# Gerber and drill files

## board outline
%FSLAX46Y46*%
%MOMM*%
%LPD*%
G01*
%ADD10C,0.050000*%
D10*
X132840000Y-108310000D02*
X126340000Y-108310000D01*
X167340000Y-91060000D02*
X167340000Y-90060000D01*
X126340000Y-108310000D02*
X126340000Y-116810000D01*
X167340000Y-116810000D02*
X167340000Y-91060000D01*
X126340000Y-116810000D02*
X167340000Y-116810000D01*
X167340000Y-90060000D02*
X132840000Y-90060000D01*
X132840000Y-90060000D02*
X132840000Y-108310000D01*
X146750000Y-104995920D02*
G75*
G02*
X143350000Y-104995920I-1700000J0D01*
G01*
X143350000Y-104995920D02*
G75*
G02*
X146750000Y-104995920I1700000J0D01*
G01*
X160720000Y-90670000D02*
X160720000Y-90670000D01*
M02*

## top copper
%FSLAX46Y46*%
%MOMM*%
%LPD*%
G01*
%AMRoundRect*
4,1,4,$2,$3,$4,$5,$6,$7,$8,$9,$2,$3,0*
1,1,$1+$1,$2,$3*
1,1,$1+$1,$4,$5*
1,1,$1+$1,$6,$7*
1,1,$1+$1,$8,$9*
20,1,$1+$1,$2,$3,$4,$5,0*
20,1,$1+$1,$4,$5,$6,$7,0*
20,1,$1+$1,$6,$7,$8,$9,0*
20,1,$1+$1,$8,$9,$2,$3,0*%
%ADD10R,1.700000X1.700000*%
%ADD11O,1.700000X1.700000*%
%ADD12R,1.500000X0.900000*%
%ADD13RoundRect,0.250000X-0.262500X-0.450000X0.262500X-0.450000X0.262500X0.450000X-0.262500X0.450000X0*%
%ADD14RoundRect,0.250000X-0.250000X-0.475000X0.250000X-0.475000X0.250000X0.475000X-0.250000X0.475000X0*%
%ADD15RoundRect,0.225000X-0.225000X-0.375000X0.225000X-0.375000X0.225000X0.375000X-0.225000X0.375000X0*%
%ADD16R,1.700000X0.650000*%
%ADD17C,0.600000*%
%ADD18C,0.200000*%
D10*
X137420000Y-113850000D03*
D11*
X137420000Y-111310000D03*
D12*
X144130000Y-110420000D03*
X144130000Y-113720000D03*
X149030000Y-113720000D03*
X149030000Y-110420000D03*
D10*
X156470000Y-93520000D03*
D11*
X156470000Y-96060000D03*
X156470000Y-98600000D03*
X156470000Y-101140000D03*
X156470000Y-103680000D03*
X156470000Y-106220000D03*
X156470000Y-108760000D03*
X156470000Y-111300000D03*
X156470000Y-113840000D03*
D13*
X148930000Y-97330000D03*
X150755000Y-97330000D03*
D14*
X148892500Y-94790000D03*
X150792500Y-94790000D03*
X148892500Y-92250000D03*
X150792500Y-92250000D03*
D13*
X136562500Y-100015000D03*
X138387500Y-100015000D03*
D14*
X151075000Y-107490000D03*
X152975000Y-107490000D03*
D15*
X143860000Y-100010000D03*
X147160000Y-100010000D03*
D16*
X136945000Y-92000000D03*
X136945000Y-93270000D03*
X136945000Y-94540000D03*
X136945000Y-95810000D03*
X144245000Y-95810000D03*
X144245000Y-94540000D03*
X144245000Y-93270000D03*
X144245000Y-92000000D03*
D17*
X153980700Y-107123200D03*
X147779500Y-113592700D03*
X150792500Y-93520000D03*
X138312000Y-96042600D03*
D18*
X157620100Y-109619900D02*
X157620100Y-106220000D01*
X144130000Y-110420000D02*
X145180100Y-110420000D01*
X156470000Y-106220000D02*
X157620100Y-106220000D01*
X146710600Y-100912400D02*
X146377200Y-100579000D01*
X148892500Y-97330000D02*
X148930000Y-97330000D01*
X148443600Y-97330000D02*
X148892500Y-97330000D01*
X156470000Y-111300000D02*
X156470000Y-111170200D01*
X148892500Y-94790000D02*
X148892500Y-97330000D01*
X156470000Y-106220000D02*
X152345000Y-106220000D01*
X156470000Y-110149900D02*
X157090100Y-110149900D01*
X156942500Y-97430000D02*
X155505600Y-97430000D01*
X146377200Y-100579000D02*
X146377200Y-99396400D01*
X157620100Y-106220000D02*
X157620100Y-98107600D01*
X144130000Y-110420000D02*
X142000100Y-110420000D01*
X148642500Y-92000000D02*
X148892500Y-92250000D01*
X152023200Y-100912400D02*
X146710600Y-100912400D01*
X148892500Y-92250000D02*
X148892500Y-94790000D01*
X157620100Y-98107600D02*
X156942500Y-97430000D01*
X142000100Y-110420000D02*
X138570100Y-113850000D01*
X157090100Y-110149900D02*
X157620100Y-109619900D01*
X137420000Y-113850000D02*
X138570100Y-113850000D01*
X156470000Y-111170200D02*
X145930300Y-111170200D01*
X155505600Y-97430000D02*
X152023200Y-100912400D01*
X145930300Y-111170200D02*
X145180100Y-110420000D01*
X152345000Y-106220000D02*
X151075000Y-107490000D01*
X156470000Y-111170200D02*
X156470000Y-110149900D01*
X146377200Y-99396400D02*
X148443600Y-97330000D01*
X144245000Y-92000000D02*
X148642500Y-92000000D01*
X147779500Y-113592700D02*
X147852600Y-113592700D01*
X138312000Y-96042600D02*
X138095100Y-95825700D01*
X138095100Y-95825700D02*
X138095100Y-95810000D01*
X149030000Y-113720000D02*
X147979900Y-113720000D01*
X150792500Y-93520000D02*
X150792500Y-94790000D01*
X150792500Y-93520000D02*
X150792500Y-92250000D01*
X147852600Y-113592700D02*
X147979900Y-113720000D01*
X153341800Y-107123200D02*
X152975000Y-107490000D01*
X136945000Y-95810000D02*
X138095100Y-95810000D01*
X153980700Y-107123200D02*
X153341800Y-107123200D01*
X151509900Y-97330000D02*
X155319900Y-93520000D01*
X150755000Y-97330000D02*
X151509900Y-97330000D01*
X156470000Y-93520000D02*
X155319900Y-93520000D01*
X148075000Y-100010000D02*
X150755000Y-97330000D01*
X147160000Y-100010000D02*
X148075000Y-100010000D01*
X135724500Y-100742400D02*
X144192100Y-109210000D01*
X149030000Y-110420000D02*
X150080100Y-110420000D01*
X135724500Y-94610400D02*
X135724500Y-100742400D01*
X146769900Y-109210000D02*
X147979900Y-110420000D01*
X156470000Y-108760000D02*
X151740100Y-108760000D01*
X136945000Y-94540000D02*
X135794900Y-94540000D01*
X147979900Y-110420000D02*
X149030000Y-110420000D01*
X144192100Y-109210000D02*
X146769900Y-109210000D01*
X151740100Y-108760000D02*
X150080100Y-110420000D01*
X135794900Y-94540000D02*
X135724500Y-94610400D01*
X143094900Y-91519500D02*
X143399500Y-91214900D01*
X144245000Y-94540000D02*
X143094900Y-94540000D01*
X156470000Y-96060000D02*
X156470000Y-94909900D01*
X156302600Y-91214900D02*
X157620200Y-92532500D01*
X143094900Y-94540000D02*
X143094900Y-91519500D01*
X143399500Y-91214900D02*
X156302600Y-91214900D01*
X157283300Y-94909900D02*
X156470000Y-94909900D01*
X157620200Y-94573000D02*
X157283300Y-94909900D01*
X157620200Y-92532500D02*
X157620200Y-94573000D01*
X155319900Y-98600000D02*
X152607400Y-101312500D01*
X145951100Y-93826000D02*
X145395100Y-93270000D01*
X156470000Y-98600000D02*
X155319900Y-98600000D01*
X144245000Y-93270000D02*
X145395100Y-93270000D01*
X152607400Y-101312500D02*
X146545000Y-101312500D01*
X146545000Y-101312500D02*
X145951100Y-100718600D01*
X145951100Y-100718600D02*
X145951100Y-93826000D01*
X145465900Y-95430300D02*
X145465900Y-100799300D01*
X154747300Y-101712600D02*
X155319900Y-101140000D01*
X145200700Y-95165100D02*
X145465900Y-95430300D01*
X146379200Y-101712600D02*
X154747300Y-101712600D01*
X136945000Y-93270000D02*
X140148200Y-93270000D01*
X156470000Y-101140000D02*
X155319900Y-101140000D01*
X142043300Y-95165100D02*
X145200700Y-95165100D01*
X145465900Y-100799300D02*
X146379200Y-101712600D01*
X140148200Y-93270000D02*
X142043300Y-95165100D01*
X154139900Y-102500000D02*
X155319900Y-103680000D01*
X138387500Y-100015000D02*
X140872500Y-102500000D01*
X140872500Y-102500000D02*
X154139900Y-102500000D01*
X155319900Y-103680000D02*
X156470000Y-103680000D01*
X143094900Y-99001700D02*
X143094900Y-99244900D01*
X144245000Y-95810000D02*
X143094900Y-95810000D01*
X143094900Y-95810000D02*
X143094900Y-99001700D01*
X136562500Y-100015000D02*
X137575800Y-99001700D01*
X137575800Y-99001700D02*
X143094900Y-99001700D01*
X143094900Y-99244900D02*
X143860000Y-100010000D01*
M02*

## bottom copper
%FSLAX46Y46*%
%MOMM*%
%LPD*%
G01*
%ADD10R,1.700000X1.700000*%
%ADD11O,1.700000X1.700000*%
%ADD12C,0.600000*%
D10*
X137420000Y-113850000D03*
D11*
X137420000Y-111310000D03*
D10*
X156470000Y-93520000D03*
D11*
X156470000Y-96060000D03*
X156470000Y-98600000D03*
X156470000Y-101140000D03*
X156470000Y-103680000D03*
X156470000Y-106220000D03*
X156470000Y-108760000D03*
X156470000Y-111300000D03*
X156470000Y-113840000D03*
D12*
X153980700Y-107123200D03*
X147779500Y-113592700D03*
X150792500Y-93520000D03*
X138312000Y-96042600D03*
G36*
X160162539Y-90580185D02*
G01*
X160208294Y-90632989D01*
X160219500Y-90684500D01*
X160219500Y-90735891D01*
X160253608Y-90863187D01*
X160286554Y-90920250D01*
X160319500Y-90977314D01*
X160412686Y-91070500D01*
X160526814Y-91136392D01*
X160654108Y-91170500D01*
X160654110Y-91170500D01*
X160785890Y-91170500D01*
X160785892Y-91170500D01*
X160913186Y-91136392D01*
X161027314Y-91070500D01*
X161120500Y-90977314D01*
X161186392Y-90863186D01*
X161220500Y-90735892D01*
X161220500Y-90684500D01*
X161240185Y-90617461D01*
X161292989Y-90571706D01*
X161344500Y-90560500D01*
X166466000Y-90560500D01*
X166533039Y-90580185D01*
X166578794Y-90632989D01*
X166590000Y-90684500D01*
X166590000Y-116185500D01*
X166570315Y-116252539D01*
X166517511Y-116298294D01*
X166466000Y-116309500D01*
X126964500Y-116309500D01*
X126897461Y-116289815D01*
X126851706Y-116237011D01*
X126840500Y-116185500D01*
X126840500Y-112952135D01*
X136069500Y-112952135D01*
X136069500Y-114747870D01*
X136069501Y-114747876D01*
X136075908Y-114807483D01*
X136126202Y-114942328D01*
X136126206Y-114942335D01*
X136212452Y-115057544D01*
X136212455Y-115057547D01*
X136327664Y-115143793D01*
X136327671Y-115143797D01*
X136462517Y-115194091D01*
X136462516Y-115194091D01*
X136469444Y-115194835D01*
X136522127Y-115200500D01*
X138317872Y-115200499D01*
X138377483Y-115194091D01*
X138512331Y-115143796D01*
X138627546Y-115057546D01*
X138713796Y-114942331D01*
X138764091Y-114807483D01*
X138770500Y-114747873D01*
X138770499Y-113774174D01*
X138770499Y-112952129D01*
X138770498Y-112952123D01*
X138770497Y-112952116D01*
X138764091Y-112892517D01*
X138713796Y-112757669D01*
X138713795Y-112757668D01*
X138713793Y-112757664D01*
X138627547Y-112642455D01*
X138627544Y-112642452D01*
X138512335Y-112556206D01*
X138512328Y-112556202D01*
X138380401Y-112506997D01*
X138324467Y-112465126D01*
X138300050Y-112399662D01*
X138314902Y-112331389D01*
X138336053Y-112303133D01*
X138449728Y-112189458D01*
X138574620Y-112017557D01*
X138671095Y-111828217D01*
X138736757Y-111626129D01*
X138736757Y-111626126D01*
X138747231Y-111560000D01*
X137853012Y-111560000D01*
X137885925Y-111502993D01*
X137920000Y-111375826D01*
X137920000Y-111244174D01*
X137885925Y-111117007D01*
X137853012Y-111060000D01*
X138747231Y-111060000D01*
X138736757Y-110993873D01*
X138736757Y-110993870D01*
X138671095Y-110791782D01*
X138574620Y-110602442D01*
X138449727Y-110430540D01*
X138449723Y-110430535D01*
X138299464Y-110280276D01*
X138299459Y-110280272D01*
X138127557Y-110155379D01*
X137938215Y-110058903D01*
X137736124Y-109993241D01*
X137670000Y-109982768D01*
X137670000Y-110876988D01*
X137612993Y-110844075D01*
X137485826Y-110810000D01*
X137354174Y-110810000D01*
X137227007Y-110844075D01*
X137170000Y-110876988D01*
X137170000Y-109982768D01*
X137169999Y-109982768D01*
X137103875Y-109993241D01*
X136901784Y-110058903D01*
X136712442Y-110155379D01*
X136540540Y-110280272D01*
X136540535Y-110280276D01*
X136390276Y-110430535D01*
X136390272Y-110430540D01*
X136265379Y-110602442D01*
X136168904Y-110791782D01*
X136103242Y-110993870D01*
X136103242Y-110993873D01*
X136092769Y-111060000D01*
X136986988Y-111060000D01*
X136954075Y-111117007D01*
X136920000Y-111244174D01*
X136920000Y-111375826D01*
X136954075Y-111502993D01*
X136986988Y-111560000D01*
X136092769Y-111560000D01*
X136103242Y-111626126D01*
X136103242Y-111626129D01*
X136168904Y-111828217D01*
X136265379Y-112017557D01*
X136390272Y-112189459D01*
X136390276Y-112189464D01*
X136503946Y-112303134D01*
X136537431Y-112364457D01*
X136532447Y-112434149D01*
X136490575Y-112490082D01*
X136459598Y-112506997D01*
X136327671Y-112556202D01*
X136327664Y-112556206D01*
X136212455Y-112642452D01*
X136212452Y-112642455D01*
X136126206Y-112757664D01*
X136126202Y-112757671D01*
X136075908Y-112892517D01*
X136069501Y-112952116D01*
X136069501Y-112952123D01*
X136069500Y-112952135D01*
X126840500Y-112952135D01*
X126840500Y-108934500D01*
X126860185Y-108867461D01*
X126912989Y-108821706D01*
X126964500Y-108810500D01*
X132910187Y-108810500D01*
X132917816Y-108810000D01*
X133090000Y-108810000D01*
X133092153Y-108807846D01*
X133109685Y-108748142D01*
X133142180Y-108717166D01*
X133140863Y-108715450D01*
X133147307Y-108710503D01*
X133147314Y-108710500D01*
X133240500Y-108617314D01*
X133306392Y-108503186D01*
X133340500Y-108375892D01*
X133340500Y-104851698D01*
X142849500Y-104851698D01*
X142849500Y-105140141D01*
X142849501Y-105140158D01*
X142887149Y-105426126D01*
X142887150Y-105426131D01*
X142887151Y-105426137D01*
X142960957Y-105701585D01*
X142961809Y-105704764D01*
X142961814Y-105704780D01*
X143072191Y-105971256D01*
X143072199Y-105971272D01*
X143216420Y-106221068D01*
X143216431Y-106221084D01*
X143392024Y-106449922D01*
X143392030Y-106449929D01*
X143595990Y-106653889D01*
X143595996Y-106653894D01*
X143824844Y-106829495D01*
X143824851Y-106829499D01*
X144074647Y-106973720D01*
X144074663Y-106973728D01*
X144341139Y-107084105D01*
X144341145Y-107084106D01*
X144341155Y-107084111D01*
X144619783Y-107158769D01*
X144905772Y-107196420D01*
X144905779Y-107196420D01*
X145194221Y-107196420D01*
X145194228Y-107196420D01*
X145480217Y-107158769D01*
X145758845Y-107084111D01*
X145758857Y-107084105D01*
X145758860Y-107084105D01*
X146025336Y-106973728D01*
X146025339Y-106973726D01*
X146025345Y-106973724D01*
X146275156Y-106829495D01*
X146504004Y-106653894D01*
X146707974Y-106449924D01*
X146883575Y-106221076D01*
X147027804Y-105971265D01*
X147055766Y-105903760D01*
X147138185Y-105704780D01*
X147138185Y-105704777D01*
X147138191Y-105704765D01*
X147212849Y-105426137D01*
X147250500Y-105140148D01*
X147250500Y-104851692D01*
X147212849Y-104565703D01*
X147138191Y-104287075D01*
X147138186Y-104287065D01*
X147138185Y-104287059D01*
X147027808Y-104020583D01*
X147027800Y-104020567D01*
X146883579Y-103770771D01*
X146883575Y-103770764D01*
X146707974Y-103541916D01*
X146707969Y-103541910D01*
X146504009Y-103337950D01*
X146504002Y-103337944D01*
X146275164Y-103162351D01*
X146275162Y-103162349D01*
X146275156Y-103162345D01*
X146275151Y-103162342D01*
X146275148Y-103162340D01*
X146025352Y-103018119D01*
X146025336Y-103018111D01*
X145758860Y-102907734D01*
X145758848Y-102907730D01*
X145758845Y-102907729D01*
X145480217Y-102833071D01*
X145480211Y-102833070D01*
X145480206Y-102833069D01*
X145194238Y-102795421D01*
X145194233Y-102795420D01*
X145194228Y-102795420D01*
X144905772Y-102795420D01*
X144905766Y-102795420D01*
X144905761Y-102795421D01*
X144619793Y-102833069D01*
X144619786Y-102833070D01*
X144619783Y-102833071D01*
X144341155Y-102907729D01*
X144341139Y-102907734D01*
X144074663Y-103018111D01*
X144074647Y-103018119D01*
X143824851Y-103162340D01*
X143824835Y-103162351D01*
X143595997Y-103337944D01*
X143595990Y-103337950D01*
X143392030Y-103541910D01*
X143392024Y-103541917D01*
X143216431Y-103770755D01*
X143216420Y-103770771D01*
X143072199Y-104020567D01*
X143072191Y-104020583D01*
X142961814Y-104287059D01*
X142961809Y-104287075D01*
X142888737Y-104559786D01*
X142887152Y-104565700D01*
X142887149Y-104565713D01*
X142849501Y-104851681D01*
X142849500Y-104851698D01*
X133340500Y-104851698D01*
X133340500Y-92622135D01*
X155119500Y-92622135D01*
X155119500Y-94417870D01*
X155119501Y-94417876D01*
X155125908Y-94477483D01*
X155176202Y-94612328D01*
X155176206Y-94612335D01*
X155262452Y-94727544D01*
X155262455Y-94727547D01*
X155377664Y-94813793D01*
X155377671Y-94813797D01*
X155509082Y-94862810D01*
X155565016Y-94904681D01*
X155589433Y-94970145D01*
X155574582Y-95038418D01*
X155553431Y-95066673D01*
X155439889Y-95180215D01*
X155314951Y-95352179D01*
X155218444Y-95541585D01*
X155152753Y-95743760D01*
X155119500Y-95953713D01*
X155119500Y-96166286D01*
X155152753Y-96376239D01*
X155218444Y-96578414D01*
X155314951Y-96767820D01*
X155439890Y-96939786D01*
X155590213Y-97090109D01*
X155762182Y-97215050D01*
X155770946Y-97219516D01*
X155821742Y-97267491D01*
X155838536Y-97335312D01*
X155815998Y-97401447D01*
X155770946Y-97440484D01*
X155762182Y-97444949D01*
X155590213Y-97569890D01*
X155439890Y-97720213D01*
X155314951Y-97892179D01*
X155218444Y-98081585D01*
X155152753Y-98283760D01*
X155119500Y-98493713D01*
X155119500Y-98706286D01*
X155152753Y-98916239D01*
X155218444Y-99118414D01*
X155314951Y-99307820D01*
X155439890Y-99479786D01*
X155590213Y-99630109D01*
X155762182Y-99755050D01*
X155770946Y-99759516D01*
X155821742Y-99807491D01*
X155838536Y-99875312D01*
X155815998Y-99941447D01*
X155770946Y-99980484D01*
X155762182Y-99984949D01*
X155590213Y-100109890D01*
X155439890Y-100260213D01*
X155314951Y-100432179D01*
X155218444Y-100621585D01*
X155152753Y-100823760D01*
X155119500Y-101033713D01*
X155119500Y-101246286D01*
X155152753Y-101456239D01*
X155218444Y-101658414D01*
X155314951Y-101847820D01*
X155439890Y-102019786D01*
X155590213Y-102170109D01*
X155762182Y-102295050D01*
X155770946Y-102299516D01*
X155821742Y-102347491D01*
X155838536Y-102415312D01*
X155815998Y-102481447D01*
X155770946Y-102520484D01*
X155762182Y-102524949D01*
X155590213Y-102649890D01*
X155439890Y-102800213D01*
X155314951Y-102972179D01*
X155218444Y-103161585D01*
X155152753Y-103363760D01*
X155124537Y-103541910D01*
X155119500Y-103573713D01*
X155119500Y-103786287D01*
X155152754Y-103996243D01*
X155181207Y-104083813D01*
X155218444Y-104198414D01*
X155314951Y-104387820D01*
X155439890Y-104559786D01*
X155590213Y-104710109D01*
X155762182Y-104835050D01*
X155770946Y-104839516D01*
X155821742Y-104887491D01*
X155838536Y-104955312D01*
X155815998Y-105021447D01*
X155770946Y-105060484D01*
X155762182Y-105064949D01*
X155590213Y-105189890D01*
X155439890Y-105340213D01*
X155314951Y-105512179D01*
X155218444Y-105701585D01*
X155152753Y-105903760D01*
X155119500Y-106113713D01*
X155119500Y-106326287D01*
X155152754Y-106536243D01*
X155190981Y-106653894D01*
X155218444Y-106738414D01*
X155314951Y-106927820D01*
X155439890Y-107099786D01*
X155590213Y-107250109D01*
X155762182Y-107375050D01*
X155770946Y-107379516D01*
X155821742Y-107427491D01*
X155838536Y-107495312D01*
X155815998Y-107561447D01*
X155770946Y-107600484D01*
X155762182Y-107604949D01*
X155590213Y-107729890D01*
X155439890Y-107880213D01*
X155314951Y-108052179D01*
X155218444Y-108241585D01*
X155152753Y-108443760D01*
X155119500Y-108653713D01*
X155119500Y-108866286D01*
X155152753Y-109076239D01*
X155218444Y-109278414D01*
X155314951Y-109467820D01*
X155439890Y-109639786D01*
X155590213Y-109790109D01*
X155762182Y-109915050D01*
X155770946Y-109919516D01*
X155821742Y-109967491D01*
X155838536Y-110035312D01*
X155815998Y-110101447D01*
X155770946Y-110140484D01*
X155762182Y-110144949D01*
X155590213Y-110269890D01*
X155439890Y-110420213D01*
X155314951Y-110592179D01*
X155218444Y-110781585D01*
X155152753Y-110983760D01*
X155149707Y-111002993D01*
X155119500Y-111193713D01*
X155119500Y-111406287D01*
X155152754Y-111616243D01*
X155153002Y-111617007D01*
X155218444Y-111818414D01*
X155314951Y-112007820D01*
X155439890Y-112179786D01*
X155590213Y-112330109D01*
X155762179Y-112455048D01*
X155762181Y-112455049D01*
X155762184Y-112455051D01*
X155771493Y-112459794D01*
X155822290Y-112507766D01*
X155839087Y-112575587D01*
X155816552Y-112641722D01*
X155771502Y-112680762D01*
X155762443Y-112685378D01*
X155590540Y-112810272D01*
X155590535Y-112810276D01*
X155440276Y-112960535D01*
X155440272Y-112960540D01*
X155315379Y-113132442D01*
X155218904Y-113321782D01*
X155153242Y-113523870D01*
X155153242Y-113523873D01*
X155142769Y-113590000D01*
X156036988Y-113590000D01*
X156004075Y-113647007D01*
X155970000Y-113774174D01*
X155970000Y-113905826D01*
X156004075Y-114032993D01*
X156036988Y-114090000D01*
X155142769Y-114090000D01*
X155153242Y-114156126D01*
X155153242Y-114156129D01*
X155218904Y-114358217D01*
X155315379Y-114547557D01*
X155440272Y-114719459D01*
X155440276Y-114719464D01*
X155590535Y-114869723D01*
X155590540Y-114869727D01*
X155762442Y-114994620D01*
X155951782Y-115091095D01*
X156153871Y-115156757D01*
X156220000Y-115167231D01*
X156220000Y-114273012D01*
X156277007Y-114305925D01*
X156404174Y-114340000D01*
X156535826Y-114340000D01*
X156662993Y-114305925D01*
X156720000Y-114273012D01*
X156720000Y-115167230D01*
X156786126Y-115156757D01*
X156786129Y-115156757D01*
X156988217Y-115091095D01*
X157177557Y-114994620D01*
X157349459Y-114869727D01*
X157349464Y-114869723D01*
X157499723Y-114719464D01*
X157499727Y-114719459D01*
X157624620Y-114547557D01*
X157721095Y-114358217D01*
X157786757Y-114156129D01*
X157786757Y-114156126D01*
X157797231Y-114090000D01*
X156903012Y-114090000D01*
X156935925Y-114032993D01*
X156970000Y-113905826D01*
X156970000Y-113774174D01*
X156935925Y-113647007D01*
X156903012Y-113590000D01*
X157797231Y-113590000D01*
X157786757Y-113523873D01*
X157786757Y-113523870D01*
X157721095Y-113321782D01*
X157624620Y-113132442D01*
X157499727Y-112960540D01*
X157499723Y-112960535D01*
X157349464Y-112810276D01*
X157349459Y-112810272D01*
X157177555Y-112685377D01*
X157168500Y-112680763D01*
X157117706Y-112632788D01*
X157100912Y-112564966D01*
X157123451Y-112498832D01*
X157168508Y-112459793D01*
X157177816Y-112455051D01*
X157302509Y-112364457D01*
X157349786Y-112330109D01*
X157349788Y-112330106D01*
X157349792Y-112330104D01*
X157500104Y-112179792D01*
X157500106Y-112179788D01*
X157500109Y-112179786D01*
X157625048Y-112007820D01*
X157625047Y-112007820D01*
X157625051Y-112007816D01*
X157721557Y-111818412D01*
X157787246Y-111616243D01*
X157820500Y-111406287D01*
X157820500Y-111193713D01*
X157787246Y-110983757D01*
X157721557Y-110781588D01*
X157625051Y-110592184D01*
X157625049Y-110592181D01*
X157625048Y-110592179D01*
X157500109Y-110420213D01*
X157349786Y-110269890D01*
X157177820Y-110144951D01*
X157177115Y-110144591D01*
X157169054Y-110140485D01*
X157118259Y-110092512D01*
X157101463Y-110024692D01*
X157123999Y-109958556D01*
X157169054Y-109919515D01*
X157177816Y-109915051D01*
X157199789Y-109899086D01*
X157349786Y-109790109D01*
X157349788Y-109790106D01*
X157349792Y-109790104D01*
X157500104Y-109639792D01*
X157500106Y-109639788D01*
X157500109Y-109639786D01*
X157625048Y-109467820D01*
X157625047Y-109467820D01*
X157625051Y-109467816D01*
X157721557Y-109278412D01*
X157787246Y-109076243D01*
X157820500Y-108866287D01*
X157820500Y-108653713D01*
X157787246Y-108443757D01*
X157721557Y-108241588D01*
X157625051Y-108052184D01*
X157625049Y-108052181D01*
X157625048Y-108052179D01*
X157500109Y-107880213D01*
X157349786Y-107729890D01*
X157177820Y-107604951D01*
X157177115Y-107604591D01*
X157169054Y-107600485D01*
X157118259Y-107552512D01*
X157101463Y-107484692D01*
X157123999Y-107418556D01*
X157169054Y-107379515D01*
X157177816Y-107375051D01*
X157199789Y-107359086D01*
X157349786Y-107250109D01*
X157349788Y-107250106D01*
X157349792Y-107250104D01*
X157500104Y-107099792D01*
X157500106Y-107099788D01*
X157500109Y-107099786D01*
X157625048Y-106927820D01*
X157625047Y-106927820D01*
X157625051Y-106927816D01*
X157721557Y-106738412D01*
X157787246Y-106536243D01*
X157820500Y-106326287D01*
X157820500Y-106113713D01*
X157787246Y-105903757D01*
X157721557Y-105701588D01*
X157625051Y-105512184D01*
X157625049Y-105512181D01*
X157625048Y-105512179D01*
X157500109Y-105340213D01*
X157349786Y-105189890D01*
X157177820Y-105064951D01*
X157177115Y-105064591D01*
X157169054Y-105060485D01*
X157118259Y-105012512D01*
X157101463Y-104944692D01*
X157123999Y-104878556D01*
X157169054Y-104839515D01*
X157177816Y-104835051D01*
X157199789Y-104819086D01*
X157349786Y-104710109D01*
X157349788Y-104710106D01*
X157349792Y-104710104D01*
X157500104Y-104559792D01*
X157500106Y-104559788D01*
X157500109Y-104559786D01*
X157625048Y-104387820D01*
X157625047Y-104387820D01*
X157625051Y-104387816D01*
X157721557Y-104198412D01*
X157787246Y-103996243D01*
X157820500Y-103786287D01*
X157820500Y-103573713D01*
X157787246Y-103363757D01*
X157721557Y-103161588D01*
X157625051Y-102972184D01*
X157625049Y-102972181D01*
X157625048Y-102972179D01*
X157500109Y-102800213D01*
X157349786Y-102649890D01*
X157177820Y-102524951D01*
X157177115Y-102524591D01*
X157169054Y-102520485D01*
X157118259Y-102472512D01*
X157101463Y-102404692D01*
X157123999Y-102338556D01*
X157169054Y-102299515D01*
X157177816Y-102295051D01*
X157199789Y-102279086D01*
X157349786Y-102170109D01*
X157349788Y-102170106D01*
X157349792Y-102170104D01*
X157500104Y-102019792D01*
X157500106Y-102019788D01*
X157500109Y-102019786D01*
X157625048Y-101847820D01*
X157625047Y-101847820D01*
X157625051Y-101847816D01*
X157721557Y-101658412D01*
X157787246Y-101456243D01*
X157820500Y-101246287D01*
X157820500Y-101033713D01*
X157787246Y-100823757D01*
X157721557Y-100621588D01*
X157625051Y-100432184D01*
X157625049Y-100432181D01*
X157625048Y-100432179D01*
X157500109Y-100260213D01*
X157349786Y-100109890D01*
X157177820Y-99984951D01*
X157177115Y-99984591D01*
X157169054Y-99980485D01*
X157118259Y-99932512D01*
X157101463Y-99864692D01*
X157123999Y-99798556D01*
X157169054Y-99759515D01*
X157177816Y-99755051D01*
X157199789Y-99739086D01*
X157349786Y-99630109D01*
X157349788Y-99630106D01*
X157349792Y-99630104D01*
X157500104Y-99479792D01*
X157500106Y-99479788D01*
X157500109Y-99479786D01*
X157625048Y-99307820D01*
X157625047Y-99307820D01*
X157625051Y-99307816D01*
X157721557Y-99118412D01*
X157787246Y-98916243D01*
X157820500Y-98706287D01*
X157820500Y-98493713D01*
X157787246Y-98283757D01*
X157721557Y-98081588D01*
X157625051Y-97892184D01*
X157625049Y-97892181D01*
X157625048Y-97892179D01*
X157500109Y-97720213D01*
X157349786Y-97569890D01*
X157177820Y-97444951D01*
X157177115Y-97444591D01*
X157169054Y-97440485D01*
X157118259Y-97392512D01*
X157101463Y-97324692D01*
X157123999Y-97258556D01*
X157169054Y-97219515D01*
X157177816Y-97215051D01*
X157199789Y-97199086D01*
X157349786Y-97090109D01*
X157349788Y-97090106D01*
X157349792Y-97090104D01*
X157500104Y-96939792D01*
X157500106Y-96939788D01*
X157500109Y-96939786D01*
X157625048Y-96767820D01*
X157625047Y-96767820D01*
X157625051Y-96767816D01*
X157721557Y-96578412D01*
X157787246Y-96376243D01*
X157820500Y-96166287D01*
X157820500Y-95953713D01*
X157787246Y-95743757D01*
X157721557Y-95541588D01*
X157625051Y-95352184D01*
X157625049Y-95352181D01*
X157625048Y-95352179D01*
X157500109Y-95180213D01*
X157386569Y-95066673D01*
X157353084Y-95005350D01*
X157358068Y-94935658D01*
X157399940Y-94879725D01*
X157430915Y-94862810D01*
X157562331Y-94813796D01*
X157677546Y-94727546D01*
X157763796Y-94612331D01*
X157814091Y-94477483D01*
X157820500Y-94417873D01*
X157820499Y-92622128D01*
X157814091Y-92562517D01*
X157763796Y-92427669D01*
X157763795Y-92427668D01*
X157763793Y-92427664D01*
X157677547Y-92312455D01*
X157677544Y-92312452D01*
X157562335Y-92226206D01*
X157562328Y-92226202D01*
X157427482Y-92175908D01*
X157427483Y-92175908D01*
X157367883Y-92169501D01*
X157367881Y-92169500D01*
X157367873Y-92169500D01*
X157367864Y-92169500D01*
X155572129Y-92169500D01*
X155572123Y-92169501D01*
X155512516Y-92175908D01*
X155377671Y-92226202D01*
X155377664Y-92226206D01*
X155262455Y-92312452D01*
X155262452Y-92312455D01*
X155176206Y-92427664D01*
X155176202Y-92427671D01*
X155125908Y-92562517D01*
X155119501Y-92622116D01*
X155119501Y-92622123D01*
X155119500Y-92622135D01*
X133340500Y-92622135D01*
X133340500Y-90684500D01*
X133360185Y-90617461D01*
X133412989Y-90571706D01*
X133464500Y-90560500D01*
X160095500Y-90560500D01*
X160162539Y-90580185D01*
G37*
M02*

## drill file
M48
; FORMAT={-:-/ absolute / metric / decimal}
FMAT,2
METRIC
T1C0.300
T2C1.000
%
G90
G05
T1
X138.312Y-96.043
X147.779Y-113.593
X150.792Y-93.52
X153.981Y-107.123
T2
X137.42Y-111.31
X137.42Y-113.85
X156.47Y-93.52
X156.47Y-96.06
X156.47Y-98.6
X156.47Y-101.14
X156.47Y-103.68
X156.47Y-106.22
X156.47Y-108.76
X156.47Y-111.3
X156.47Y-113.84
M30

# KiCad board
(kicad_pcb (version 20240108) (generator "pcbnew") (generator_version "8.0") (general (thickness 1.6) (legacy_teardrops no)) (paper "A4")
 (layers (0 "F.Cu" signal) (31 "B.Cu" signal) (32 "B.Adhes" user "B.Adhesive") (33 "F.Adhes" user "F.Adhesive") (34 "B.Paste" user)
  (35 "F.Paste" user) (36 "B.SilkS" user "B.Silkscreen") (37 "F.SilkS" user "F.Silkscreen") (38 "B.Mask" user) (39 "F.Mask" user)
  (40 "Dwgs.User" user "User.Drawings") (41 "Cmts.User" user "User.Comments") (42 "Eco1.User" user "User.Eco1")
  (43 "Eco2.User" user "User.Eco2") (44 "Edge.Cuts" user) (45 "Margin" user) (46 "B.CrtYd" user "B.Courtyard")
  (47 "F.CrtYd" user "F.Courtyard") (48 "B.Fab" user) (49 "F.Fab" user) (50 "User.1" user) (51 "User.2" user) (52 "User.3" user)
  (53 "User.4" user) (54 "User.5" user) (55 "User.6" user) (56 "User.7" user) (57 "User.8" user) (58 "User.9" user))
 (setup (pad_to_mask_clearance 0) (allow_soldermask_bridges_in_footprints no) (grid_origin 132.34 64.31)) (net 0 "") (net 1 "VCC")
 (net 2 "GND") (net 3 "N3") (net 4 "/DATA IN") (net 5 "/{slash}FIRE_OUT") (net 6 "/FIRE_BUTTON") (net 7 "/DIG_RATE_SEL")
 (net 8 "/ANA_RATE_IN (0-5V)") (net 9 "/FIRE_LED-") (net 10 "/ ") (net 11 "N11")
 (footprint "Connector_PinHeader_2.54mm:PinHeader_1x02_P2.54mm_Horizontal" (layer "F.Cu") (at 137.42 113.85 180)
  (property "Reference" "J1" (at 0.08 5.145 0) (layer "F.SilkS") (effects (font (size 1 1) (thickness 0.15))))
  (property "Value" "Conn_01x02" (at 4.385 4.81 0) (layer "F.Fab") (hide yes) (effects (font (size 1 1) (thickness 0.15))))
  (pad "1" thru_hole rect (at 0 0 180) (size 1.7 1.7) (drill 1) (layers "*.Cu" "*.Mask") (remove_unused_layers no) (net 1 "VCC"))
  (pad "2" thru_hole oval (at 0 2.54 180) (size 1.7 1.7) (drill 1) (layers "*.Cu" "*.Mask") (remove_unused_layers no) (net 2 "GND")))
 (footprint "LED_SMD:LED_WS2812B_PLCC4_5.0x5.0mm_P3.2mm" (layer "F.Cu") (at 146.58 112.07)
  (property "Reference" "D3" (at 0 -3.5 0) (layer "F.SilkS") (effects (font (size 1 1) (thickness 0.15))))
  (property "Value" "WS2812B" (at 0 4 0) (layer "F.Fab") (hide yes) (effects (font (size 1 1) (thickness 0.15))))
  (pad "1" smd rect (at -2.45 -1.65) (size 1.5 0.9) (layers "F.Cu" "F.Paste" "F.Mask") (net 1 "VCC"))
  (pad "2" smd rect (at -2.45 1.65) (size 1.5 0.9) (layers "F.Cu" "F.Paste" "F.Mask") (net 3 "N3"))
  (pad "3" smd rect (at 2.45 1.65) (size 1.5 0.9) (layers "F.Cu" "F.Paste" "F.Mask") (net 2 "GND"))
  (pad "4" smd rect (at 2.45 -1.65) (size 1.5 0.9) (layers "F.Cu" "F.Paste" "F.Mask") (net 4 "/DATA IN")))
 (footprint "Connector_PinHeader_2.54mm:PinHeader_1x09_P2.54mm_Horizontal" (layer "F.Cu") (at 156.47 93.52)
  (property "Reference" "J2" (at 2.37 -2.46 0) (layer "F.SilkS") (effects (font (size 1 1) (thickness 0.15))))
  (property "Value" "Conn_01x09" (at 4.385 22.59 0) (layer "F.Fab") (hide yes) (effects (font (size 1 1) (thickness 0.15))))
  (pad "1" thru_hole rect (at 0 0) (size 1.7 1.7) (drill 1) (layers "*.Cu" "*.Mask") (remove_unused_layers no) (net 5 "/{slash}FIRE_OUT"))
  (pad "2" thru_hole oval (at 0 2.54) (size 1.7 1.7) (drill 1) (layers "*.Cu" "*.Mask") (remove_unused_layers no) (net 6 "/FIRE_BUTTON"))
  (pad "3" thru_hole oval (at 0 5.08) (size 1.7 1.7) (drill 1) (layers "*.Cu" "*.Mask") (remove_unused_layers no) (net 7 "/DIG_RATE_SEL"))
  (pad "4" thru_hole oval (at 0 7.62) (size 1.7 1.7) (drill 1) (layers "*.Cu" "*.Mask") (remove_unused_layers no)
   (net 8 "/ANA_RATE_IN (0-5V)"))
  (pad "5" thru_hole oval (at 0 10.16) (size 1.7 1.7) (drill 1) (layers "*.Cu" "*.Mask") (remove_unused_layers no) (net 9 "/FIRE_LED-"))
  (pad "6" thru_hole oval (at 0 12.7) (size 1.7 1.7) (drill 1) (layers "*.Cu" "*.Mask") (remove_unused_layers no) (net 1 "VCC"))
  (pad "7" thru_hole oval (at 0 15.24) (size 1.7 1.7) (drill 1) (layers "*.Cu" "*.Mask") (remove_unused_layers no) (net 4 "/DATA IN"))
  (pad "8" thru_hole oval (at 0 17.78) (size 1.7 1.7) (drill 1) (layers "*.Cu" "*.Mask") (remove_unused_layers no) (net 1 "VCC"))
  (pad "9" thru_hole oval (at 0 20.32) (size 1.7 1.7) (drill 1) (layers "*.Cu" "*.Mask") (remove_unused_layers no) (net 2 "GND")))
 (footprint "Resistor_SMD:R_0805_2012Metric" (layer "F.Cu") (at 149.8425 97.33)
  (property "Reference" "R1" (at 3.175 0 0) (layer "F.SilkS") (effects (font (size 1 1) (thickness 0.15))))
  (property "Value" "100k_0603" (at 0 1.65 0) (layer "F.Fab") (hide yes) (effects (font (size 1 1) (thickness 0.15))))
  (pad "1" smd roundrect (at -0.9125 0) (size 1.025 1.4) (layers "F.Cu" "F.Paste" "F.Mask") (roundrect_rratio 0.243902439) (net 1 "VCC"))
  (pad "2" smd roundrect (at 0.9125 0) (size 1.025 1.4) (layers "F.Cu" "F.Paste" "F.Mask") (roundrect_rratio 0.243902439)
   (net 5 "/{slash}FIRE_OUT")))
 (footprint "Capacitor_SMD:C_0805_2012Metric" (layer "F.Cu") (at 149.8425 94.79)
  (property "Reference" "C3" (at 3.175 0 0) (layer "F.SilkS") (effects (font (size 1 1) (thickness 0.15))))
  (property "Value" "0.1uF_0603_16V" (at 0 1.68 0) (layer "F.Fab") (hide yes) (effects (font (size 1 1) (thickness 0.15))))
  (pad "1" smd roundrect (at -0.95 0) (size 1 1.45) (layers "F.Cu" "F.Paste" "F.Mask") (roundrect_rratio 0.25) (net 1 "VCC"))
  (pad "2" smd roundrect (at 0.95 0) (size 1 1.45) (layers "F.Cu" "F.Paste" "F.Mask") (roundrect_rratio 0.25) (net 2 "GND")))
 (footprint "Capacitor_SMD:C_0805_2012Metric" (layer "F.Cu") (at 149.8425 92.25)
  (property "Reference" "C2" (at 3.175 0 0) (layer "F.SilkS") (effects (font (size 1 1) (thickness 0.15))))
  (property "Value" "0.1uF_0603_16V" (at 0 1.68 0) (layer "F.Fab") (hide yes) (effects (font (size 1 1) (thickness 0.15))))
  (pad "1" smd roundrect (at -0.95 0) (size 1 1.45) (layers "F.Cu" "F.Paste" "F.Mask") (roundrect_rratio 0.25) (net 1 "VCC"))
  (pad "2" smd roundrect (at 0.95 0) (size 1 1.45) (layers "F.Cu" "F.Paste" "F.Mask") (roundrect_rratio 0.25) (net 2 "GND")))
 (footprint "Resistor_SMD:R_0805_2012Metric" (layer "F.Cu") (at 137.475 100.015)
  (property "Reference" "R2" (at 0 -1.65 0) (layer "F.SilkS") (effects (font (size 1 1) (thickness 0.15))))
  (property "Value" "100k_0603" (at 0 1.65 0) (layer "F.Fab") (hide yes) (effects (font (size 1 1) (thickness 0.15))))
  (pad "1" smd roundrect (at -0.9125 0) (size 1.025 1.4) (layers "F.Cu" "F.Paste" "F.Mask") (roundrect_rratio 0.243902439) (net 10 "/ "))
  (pad "2" smd roundrect (at 0.9125 0) (size 1.025 1.4) (layers "F.Cu" "F.Paste" "F.Mask") (roundrect_rratio 0.243902439)
   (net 9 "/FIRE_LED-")))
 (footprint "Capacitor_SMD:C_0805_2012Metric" (layer "F.Cu") (at 152.025 107.49)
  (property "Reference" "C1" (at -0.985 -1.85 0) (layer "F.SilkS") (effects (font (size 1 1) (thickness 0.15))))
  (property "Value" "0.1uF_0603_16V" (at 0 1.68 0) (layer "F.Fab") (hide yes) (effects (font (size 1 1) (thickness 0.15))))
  (pad "1" smd roundrect (at -0.95 0) (size 1 1.45) (layers "F.Cu" "F.Paste" "F.Mask") (roundrect_rratio 0.25) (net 1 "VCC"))
  (pad "2" smd roundrect (at 0.95 0) (size 1 1.45) (layers "F.Cu" "F.Paste" "F.Mask") (roundrect_rratio 0.25) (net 2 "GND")))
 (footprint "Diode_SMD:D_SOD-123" (layer "F.Cu") (at 145.51 100.01)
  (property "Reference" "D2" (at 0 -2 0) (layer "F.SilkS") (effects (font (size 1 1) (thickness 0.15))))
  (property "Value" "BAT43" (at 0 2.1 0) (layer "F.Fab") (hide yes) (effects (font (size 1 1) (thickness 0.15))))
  (pad "1" smd roundrect (at -1.65 0) (size 0.9 1.2) (layers "F.Cu" "F.Paste" "F.Mask") (roundrect_rratio 0.25) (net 10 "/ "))
  (pad "2" smd roundrect (at 1.65 0) (size 0.9 1.2) (layers "F.Cu" "F.Paste" "F.Mask") (roundrect_rratio 0.25) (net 5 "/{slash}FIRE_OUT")))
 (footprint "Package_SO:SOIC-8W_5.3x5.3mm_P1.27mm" (layer "F.Cu") (at 140.595 93.905)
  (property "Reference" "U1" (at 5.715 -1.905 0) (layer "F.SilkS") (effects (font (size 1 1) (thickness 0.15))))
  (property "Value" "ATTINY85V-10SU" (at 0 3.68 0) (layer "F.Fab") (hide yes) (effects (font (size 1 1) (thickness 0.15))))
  (pad "1" smd rect (at -3.65 -1.905) (size 1.7 0.65) (layers "F.Cu" "F.Paste" "F.Mask") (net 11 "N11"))
  (pad "2" smd rect (at -3.65 -0.635) (size 1.7 0.65) (layers "F.Cu" "F.Paste" "F.Mask") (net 8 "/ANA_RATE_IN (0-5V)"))
  (pad "3" smd rect (at -3.65 0.635) (size 1.7 0.65) (layers "F.Cu" "F.Paste" "F.Mask") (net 4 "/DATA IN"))
  (pad "4" smd rect (at -3.65 1.905) (size 1.7 0.65) (layers "F.Cu" "F.Paste" "F.Mask") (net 2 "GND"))
  (pad "5" smd rect (at 3.65 1.905) (size 1.7 0.65) (layers "F.Cu" "F.Paste" "F.Mask") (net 10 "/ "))
  (pad "6" smd rect (at 3.65 0.635) (size 1.7 0.65) (layers "F.Cu" "F.Paste" "F.Mask") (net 6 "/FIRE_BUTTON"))
  (pad "7" smd rect (at 3.65 -0.635) (size 1.7 0.65) (layers "F.Cu" "F.Paste" "F.Mask") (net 7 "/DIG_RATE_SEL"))
  (pad "8" smd rect (at 3.65 -1.905) (size 1.7 0.65) (layers "F.Cu" "F.Paste" "F.Mask") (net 1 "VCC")))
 (gr_line (start 132.84 108.31) (end 126.34 108.31) (stroke (width 0.05) (type default)) (layer "Edge.Cuts"))
 (gr_line (start 167.34 91.06) (end 167.34 90.06) (stroke (width 0.05) (type default)) (layer "Edge.Cuts"))
 (gr_line (start 126.34 108.31) (end 126.34 116.81) (stroke (width 0.05) (type default)) (layer "Edge.Cuts"))
 (gr_line (start 167.34 116.81) (end 167.34 91.06) (stroke (width 0.05) (type default)) (layer "Edge.Cuts"))
 (gr_line (start 126.34 116.81) (end 167.34 116.81) (stroke (width 0.05) (type default)) (layer "Edge.Cuts"))
 (gr_line (start 167.34 90.06) (end 132.84 90.06) (stroke (width 0.05) (type default)) (layer "Edge.Cuts"))
 (gr_line (start 132.84 90.06) (end 132.84 108.31) (stroke (width 0.05) (type default)) (layer "Edge.Cuts"))
 (gr_circle (center 145.05 104.99592) (end 146.75 104.99592) (stroke (width 0.05) (type default)) (fill none) (layer "Edge.Cuts"))
 (gr_line (start 160.72 90.67) (end 160.72 90.67) (stroke (width 0.05) (type default)) (layer "Edge.Cuts"))
 (segment (start 157.6201 109.6199) (end 157.6201 106.22) (width 0.2) (layer "F.Cu") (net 1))
 (segment (start 144.13 110.42) (end 145.1801 110.42) (width 0.2) (layer "F.Cu") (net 1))
 (segment (start 156.47 106.22) (end 157.6201 106.22) (width 0.2) (layer "F.Cu") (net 1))
 (segment (start 146.7106 100.9124) (end 146.3772 100.579) (width 0.2) (layer "F.Cu") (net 1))
 (segment (start 148.8925 97.33) (end 148.93 97.33) (width 0.2) (layer "F.Cu") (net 1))
 (segment (start 148.4436 97.33) (end 148.8925 97.33) (width 0.2) (layer "F.Cu") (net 1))
 (segment (start 156.47 111.3) (end 156.47 111.1702) (width 0.2) (layer "F.Cu") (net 1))
 (segment (start 148.8925 94.79) (end 148.8925 97.33) (width 0.2) (layer "F.Cu") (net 1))
 (segment (start 156.47 106.22) (end 152.345 106.22) (width 0.2) (layer "F.Cu") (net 1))
 (segment (start 156.47 110.1499) (end 157.0901 110.1499) (width 0.2) (layer "F.Cu") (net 1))
 (segment (start 156.9425 97.43) (end 155.5056 97.43) (width 0.2) (layer "F.Cu") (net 1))
 (segment (start 146.3772 100.579) (end 146.3772 99.3964) (width 0.2) (layer "F.Cu") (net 1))
 (segment (start 157.6201 106.22) (end 157.6201 98.1076) (width 0.2) (layer "F.Cu") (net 1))
 (segment (start 144.13 110.42) (end 142.0001 110.42) (width 0.2) (layer "F.Cu") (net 1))
 (segment (start 148.6425 92) (end 148.8925 92.25) (width 0.2) (layer "F.Cu") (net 1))
 (segment (start 152.0232 100.9124) (end 146.7106 100.9124) (width 0.2) (layer "F.Cu") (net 1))
 (segment (start 148.8925 92.25) (end 148.8925 94.79) (width 0.2) (layer "F.Cu") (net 1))
 (segment (start 157.6201 98.1076) (end 156.9425 97.43) (width 0.2) (layer "F.Cu") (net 1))
 (segment (start 142.0001 110.42) (end 138.5701 113.85) (width 0.2) (layer "F.Cu") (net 1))
 (segment (start 157.0901 110.1499) (end 157.6201 109.6199) (width 0.2) (layer "F.Cu") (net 1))
 (segment (start 137.42 113.85) (end 138.5701 113.85) (width 0.2) (layer "F.Cu") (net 1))
 (segment (start 156.47 111.1702) (end 145.9303 111.1702) (width 0.2) (layer "F.Cu") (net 1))
 (segment (start 155.5056 97.43) (end 152.0232 100.9124) (width 0.2) (layer "F.Cu") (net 1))
 (segment (start 145.9303 111.1702) (end 145.1801 110.42) (width 0.2) (layer "F.Cu") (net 1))
 (segment (start 152.345 106.22) (end 151.075 107.49) (width 0.2) (layer "F.Cu") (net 1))
 (segment (start 156.47 111.1702) (end 156.47 110.1499) (width 0.2) (layer "F.Cu") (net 1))
 (segment (start 146.3772 99.3964) (end 148.4436 97.33) (width 0.2) (layer "F.Cu") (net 1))
 (segment (start 144.245 92) (end 148.6425 92) (width 0.2) (layer "F.Cu") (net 1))
 (segment (start 147.7795 113.5927) (end 147.8526 113.5927) (width 0.2) (layer "F.Cu") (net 2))
 (segment (start 138.312 96.0426) (end 138.0951 95.8257) (width 0.2) (layer "F.Cu") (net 2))
 (segment (start 138.0951 95.8257) (end 138.0951 95.81) (width 0.2) (layer "F.Cu") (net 2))
 (segment (start 149.03 113.72) (end 147.9799 113.72) (width 0.2) (layer "F.Cu") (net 2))
 (segment (start 150.7925 93.52) (end 150.7925 94.79) (width 0.2) (layer "F.Cu") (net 2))
 (segment (start 150.7925 93.52) (end 150.7925 92.25) (width 0.2) (layer "F.Cu") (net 2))
 (segment (start 147.8526 113.5927) (end 147.9799 113.72) (width 0.2) (layer "F.Cu") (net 2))
 (segment (start 153.3418 107.1232) (end 152.975 107.49) (width 0.2) (layer "F.Cu") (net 2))
 (segment (start 136.945 95.81) (end 138.0951 95.81) (width 0.2) (layer "F.Cu") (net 2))
 (segment (start 153.9807 107.1232) (end 153.3418 107.1232) (width 0.2) (layer "F.Cu") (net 2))
 (via (at 153.9807 107.1232) (size 0.6) (drill 0.3) (layers "F.Cu" "B.Cu") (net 2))
 (via (at 147.7795 113.5927) (size 0.6) (drill 0.3) (layers "F.Cu" "B.Cu") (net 2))
 (via (at 150.7925 93.52) (size 0.6) (drill 0.3) (layers "F.Cu" "B.Cu") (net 2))
 (via (at 138.312 96.0426) (size 0.6) (drill 0.3) (layers "F.Cu" "B.Cu") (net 2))
 (segment (start 151.5099 97.33) (end 155.3199 93.52) (width 0.2) (layer "F.Cu") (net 5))
 (segment (start 150.755 97.33) (end 151.5099 97.33) (width 0.2) (layer "F.Cu") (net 5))
 (segment (start 156.47 93.52) (end 155.3199 93.52) (width 0.2) (layer "F.Cu") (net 5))
 (segment (start 148.075 100.01) (end 150.755 97.33) (width 0.2) (layer "F.Cu") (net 5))
 (segment (start 147.16 100.01) (end 148.075 100.01) (width 0.2) (layer "F.Cu") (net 5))
 (segment (start 135.7245 100.7424) (end 144.1921 109.21) (width 0.2) (layer "F.Cu") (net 4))
 (segment (start 149.03 110.42) (end 150.0801 110.42) (width 0.2) (layer "F.Cu") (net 4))
 (segment (start 135.7245 94.6104) (end 135.7245 100.7424) (width 0.2) (layer "F.Cu") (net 4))
 (segment (start 146.7699 109.21) (end 147.9799 110.42) (width 0.2) (layer "F.Cu") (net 4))
 (segment (start 156.47 108.76) (end 151.7401 108.76) (width 0.2) (layer "F.Cu") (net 4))
 (segment (start 136.945 94.54) (end 135.7949 94.54) (width 0.2) (layer "F.Cu") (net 4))
 (segment (start 147.9799 110.42) (end 149.03 110.42) (width 0.2) (layer "F.Cu") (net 4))
 (segment (start 144.1921 109.21) (end 146.7699 109.21) (width 0.2) (layer "F.Cu") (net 4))
 (segment (start 151.7401 108.76) (end 150.0801 110.42) (width 0.2) (layer "F.Cu") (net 4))
 (segment (start 135.7949 94.54) (end 135.7245 94.6104) (width 0.2) (layer "F.Cu") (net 4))
 (segment (start 143.0949 91.5195) (end 143.3995 91.2149) (width 0.2) (layer "F.Cu") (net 6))
 (segment (start 144.245 94.54) (end 143.0949 94.54) (width 0.2) (layer "F.Cu") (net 6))
 (segment (start 156.47 96.06) (end 156.47 94.9099) (width 0.2) (layer "F.Cu") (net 6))
 (segment (start 156.3026 91.2149) (end 157.6202 92.5325) (width 0.2) (layer "F.Cu") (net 6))
 (segment (start 143.0949 94.54) (end 143.0949 91.5195) (width 0.2) (layer "F.Cu") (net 6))
 (segment (start 143.3995 91.2149) (end 156.3026 91.2149) (width 0.2) (layer "F.Cu") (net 6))
 (segment (start 157.2833 94.9099) (end 156.47 94.9099) (width 0.2) (layer "F.Cu") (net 6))
 (segment (start 157.6202 94.573) (end 157.2833 94.9099) (width 0.2) (layer "F.Cu") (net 6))
 (segment (start 157.6202 92.5325) (end 157.6202 94.573) (width 0.2) (layer "F.Cu") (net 6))
 (segment (start 155.3199 98.6) (end 152.6074 101.3125) (width 0.2) (layer "F.Cu") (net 7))
 (segment (start 145.9511 93.826) (end 145.3951 93.27) (width 0.2) (layer "F.Cu") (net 7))
 (segment (start 156.47 98.6) (end 155.3199 98.6) (width 0.2) (layer "F.Cu") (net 7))
 (segment (start 144.245 93.27) (end 145.3951 93.27) (width 0.2) (layer "F.Cu") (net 7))
 (segment (start 152.6074 101.3125) (end 146.545 101.3125) (width 0.2) (layer "F.Cu") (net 7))
 (segment (start 146.545 101.3125) (end 145.9511 100.7186) (width 0.2) (layer "F.Cu") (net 7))
 (segment (start 145.9511 100.7186) (end 145.9511 93.826) (width 0.2) (layer "F.Cu") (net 7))
 (segment (start 145.4659 95.4303) (end 145.4659 100.7993) (width 0.2) (layer "F.Cu") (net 8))
 (segment (start 154.7473 101.7126) (end 155.3199 101.14) (width 0.2) (layer "F.Cu") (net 8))
 (segment (start 145.2007 95.1651) (end 145.4659 95.4303) (width 0.2) (layer "F.Cu") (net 8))
 (segment (start 146.3792 101.7126) (end 154.7473 101.7126) (width 0.2) (layer "F.Cu") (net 8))
 (segment (start 136.945 93.27) (end 140.1482 93.27) (width 0.2) (layer "F.Cu") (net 8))
 (segment (start 156.47 101.14) (end 155.3199 101.14) (width 0.2) (layer "F.Cu") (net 8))
 (segment (start 142.0433 95.1651) (end 145.2007 95.1651) (width 0.2) (layer "F.Cu") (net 8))
 (segment (start 145.4659 100.7993) (end 146.3792 101.7126) (width 0.2) (layer "F.Cu") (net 8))
 (segment (start 140.1482 93.27) (end 142.0433 95.1651) (width 0.2) (layer "F.Cu") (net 8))
 (segment (start 154.1399 102.5) (end 155.3199 103.68) (width 0.2) (layer "F.Cu") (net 9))
 (segment (start 138.3875 100.015) (end 140.8725 102.5) (width 0.2) (layer "F.Cu") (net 9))
 (segment (start 140.8725 102.5) (end 154.1399 102.5) (width 0.2) (layer "F.Cu") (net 9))
 (segment (start 155.3199 103.68) (end 156.47 103.68) (width 0.2) (layer "F.Cu") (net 9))
 (segment (start 143.0949 99.0017) (end 143.0949 99.2449) (width 0.2) (layer "F.Cu") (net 10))
 (segment (start 144.245 95.81) (end 143.0949 95.81) (width 0.2) (layer "F.Cu") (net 10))
 (segment (start 143.0949 95.81) (end 143.0949 99.0017) (width 0.2) (layer "F.Cu") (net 10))
 (segment (start 136.5625 100.015) (end 137.5758 99.0017) (width 0.2) (layer "F.Cu") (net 10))
 (segment (start 137.5758 99.0017) (end 143.0949 99.0017) (width 0.2) (layer "F.Cu") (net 10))
 (segment (start 143.0949 99.2449) (end 143.86 100.01) (width 0.2) (layer "F.Cu") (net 10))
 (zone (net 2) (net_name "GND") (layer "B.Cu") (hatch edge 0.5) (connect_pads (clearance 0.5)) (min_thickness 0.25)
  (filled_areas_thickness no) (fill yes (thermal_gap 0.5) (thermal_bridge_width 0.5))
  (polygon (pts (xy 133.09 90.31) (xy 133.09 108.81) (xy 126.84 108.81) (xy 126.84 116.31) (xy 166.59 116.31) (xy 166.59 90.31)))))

